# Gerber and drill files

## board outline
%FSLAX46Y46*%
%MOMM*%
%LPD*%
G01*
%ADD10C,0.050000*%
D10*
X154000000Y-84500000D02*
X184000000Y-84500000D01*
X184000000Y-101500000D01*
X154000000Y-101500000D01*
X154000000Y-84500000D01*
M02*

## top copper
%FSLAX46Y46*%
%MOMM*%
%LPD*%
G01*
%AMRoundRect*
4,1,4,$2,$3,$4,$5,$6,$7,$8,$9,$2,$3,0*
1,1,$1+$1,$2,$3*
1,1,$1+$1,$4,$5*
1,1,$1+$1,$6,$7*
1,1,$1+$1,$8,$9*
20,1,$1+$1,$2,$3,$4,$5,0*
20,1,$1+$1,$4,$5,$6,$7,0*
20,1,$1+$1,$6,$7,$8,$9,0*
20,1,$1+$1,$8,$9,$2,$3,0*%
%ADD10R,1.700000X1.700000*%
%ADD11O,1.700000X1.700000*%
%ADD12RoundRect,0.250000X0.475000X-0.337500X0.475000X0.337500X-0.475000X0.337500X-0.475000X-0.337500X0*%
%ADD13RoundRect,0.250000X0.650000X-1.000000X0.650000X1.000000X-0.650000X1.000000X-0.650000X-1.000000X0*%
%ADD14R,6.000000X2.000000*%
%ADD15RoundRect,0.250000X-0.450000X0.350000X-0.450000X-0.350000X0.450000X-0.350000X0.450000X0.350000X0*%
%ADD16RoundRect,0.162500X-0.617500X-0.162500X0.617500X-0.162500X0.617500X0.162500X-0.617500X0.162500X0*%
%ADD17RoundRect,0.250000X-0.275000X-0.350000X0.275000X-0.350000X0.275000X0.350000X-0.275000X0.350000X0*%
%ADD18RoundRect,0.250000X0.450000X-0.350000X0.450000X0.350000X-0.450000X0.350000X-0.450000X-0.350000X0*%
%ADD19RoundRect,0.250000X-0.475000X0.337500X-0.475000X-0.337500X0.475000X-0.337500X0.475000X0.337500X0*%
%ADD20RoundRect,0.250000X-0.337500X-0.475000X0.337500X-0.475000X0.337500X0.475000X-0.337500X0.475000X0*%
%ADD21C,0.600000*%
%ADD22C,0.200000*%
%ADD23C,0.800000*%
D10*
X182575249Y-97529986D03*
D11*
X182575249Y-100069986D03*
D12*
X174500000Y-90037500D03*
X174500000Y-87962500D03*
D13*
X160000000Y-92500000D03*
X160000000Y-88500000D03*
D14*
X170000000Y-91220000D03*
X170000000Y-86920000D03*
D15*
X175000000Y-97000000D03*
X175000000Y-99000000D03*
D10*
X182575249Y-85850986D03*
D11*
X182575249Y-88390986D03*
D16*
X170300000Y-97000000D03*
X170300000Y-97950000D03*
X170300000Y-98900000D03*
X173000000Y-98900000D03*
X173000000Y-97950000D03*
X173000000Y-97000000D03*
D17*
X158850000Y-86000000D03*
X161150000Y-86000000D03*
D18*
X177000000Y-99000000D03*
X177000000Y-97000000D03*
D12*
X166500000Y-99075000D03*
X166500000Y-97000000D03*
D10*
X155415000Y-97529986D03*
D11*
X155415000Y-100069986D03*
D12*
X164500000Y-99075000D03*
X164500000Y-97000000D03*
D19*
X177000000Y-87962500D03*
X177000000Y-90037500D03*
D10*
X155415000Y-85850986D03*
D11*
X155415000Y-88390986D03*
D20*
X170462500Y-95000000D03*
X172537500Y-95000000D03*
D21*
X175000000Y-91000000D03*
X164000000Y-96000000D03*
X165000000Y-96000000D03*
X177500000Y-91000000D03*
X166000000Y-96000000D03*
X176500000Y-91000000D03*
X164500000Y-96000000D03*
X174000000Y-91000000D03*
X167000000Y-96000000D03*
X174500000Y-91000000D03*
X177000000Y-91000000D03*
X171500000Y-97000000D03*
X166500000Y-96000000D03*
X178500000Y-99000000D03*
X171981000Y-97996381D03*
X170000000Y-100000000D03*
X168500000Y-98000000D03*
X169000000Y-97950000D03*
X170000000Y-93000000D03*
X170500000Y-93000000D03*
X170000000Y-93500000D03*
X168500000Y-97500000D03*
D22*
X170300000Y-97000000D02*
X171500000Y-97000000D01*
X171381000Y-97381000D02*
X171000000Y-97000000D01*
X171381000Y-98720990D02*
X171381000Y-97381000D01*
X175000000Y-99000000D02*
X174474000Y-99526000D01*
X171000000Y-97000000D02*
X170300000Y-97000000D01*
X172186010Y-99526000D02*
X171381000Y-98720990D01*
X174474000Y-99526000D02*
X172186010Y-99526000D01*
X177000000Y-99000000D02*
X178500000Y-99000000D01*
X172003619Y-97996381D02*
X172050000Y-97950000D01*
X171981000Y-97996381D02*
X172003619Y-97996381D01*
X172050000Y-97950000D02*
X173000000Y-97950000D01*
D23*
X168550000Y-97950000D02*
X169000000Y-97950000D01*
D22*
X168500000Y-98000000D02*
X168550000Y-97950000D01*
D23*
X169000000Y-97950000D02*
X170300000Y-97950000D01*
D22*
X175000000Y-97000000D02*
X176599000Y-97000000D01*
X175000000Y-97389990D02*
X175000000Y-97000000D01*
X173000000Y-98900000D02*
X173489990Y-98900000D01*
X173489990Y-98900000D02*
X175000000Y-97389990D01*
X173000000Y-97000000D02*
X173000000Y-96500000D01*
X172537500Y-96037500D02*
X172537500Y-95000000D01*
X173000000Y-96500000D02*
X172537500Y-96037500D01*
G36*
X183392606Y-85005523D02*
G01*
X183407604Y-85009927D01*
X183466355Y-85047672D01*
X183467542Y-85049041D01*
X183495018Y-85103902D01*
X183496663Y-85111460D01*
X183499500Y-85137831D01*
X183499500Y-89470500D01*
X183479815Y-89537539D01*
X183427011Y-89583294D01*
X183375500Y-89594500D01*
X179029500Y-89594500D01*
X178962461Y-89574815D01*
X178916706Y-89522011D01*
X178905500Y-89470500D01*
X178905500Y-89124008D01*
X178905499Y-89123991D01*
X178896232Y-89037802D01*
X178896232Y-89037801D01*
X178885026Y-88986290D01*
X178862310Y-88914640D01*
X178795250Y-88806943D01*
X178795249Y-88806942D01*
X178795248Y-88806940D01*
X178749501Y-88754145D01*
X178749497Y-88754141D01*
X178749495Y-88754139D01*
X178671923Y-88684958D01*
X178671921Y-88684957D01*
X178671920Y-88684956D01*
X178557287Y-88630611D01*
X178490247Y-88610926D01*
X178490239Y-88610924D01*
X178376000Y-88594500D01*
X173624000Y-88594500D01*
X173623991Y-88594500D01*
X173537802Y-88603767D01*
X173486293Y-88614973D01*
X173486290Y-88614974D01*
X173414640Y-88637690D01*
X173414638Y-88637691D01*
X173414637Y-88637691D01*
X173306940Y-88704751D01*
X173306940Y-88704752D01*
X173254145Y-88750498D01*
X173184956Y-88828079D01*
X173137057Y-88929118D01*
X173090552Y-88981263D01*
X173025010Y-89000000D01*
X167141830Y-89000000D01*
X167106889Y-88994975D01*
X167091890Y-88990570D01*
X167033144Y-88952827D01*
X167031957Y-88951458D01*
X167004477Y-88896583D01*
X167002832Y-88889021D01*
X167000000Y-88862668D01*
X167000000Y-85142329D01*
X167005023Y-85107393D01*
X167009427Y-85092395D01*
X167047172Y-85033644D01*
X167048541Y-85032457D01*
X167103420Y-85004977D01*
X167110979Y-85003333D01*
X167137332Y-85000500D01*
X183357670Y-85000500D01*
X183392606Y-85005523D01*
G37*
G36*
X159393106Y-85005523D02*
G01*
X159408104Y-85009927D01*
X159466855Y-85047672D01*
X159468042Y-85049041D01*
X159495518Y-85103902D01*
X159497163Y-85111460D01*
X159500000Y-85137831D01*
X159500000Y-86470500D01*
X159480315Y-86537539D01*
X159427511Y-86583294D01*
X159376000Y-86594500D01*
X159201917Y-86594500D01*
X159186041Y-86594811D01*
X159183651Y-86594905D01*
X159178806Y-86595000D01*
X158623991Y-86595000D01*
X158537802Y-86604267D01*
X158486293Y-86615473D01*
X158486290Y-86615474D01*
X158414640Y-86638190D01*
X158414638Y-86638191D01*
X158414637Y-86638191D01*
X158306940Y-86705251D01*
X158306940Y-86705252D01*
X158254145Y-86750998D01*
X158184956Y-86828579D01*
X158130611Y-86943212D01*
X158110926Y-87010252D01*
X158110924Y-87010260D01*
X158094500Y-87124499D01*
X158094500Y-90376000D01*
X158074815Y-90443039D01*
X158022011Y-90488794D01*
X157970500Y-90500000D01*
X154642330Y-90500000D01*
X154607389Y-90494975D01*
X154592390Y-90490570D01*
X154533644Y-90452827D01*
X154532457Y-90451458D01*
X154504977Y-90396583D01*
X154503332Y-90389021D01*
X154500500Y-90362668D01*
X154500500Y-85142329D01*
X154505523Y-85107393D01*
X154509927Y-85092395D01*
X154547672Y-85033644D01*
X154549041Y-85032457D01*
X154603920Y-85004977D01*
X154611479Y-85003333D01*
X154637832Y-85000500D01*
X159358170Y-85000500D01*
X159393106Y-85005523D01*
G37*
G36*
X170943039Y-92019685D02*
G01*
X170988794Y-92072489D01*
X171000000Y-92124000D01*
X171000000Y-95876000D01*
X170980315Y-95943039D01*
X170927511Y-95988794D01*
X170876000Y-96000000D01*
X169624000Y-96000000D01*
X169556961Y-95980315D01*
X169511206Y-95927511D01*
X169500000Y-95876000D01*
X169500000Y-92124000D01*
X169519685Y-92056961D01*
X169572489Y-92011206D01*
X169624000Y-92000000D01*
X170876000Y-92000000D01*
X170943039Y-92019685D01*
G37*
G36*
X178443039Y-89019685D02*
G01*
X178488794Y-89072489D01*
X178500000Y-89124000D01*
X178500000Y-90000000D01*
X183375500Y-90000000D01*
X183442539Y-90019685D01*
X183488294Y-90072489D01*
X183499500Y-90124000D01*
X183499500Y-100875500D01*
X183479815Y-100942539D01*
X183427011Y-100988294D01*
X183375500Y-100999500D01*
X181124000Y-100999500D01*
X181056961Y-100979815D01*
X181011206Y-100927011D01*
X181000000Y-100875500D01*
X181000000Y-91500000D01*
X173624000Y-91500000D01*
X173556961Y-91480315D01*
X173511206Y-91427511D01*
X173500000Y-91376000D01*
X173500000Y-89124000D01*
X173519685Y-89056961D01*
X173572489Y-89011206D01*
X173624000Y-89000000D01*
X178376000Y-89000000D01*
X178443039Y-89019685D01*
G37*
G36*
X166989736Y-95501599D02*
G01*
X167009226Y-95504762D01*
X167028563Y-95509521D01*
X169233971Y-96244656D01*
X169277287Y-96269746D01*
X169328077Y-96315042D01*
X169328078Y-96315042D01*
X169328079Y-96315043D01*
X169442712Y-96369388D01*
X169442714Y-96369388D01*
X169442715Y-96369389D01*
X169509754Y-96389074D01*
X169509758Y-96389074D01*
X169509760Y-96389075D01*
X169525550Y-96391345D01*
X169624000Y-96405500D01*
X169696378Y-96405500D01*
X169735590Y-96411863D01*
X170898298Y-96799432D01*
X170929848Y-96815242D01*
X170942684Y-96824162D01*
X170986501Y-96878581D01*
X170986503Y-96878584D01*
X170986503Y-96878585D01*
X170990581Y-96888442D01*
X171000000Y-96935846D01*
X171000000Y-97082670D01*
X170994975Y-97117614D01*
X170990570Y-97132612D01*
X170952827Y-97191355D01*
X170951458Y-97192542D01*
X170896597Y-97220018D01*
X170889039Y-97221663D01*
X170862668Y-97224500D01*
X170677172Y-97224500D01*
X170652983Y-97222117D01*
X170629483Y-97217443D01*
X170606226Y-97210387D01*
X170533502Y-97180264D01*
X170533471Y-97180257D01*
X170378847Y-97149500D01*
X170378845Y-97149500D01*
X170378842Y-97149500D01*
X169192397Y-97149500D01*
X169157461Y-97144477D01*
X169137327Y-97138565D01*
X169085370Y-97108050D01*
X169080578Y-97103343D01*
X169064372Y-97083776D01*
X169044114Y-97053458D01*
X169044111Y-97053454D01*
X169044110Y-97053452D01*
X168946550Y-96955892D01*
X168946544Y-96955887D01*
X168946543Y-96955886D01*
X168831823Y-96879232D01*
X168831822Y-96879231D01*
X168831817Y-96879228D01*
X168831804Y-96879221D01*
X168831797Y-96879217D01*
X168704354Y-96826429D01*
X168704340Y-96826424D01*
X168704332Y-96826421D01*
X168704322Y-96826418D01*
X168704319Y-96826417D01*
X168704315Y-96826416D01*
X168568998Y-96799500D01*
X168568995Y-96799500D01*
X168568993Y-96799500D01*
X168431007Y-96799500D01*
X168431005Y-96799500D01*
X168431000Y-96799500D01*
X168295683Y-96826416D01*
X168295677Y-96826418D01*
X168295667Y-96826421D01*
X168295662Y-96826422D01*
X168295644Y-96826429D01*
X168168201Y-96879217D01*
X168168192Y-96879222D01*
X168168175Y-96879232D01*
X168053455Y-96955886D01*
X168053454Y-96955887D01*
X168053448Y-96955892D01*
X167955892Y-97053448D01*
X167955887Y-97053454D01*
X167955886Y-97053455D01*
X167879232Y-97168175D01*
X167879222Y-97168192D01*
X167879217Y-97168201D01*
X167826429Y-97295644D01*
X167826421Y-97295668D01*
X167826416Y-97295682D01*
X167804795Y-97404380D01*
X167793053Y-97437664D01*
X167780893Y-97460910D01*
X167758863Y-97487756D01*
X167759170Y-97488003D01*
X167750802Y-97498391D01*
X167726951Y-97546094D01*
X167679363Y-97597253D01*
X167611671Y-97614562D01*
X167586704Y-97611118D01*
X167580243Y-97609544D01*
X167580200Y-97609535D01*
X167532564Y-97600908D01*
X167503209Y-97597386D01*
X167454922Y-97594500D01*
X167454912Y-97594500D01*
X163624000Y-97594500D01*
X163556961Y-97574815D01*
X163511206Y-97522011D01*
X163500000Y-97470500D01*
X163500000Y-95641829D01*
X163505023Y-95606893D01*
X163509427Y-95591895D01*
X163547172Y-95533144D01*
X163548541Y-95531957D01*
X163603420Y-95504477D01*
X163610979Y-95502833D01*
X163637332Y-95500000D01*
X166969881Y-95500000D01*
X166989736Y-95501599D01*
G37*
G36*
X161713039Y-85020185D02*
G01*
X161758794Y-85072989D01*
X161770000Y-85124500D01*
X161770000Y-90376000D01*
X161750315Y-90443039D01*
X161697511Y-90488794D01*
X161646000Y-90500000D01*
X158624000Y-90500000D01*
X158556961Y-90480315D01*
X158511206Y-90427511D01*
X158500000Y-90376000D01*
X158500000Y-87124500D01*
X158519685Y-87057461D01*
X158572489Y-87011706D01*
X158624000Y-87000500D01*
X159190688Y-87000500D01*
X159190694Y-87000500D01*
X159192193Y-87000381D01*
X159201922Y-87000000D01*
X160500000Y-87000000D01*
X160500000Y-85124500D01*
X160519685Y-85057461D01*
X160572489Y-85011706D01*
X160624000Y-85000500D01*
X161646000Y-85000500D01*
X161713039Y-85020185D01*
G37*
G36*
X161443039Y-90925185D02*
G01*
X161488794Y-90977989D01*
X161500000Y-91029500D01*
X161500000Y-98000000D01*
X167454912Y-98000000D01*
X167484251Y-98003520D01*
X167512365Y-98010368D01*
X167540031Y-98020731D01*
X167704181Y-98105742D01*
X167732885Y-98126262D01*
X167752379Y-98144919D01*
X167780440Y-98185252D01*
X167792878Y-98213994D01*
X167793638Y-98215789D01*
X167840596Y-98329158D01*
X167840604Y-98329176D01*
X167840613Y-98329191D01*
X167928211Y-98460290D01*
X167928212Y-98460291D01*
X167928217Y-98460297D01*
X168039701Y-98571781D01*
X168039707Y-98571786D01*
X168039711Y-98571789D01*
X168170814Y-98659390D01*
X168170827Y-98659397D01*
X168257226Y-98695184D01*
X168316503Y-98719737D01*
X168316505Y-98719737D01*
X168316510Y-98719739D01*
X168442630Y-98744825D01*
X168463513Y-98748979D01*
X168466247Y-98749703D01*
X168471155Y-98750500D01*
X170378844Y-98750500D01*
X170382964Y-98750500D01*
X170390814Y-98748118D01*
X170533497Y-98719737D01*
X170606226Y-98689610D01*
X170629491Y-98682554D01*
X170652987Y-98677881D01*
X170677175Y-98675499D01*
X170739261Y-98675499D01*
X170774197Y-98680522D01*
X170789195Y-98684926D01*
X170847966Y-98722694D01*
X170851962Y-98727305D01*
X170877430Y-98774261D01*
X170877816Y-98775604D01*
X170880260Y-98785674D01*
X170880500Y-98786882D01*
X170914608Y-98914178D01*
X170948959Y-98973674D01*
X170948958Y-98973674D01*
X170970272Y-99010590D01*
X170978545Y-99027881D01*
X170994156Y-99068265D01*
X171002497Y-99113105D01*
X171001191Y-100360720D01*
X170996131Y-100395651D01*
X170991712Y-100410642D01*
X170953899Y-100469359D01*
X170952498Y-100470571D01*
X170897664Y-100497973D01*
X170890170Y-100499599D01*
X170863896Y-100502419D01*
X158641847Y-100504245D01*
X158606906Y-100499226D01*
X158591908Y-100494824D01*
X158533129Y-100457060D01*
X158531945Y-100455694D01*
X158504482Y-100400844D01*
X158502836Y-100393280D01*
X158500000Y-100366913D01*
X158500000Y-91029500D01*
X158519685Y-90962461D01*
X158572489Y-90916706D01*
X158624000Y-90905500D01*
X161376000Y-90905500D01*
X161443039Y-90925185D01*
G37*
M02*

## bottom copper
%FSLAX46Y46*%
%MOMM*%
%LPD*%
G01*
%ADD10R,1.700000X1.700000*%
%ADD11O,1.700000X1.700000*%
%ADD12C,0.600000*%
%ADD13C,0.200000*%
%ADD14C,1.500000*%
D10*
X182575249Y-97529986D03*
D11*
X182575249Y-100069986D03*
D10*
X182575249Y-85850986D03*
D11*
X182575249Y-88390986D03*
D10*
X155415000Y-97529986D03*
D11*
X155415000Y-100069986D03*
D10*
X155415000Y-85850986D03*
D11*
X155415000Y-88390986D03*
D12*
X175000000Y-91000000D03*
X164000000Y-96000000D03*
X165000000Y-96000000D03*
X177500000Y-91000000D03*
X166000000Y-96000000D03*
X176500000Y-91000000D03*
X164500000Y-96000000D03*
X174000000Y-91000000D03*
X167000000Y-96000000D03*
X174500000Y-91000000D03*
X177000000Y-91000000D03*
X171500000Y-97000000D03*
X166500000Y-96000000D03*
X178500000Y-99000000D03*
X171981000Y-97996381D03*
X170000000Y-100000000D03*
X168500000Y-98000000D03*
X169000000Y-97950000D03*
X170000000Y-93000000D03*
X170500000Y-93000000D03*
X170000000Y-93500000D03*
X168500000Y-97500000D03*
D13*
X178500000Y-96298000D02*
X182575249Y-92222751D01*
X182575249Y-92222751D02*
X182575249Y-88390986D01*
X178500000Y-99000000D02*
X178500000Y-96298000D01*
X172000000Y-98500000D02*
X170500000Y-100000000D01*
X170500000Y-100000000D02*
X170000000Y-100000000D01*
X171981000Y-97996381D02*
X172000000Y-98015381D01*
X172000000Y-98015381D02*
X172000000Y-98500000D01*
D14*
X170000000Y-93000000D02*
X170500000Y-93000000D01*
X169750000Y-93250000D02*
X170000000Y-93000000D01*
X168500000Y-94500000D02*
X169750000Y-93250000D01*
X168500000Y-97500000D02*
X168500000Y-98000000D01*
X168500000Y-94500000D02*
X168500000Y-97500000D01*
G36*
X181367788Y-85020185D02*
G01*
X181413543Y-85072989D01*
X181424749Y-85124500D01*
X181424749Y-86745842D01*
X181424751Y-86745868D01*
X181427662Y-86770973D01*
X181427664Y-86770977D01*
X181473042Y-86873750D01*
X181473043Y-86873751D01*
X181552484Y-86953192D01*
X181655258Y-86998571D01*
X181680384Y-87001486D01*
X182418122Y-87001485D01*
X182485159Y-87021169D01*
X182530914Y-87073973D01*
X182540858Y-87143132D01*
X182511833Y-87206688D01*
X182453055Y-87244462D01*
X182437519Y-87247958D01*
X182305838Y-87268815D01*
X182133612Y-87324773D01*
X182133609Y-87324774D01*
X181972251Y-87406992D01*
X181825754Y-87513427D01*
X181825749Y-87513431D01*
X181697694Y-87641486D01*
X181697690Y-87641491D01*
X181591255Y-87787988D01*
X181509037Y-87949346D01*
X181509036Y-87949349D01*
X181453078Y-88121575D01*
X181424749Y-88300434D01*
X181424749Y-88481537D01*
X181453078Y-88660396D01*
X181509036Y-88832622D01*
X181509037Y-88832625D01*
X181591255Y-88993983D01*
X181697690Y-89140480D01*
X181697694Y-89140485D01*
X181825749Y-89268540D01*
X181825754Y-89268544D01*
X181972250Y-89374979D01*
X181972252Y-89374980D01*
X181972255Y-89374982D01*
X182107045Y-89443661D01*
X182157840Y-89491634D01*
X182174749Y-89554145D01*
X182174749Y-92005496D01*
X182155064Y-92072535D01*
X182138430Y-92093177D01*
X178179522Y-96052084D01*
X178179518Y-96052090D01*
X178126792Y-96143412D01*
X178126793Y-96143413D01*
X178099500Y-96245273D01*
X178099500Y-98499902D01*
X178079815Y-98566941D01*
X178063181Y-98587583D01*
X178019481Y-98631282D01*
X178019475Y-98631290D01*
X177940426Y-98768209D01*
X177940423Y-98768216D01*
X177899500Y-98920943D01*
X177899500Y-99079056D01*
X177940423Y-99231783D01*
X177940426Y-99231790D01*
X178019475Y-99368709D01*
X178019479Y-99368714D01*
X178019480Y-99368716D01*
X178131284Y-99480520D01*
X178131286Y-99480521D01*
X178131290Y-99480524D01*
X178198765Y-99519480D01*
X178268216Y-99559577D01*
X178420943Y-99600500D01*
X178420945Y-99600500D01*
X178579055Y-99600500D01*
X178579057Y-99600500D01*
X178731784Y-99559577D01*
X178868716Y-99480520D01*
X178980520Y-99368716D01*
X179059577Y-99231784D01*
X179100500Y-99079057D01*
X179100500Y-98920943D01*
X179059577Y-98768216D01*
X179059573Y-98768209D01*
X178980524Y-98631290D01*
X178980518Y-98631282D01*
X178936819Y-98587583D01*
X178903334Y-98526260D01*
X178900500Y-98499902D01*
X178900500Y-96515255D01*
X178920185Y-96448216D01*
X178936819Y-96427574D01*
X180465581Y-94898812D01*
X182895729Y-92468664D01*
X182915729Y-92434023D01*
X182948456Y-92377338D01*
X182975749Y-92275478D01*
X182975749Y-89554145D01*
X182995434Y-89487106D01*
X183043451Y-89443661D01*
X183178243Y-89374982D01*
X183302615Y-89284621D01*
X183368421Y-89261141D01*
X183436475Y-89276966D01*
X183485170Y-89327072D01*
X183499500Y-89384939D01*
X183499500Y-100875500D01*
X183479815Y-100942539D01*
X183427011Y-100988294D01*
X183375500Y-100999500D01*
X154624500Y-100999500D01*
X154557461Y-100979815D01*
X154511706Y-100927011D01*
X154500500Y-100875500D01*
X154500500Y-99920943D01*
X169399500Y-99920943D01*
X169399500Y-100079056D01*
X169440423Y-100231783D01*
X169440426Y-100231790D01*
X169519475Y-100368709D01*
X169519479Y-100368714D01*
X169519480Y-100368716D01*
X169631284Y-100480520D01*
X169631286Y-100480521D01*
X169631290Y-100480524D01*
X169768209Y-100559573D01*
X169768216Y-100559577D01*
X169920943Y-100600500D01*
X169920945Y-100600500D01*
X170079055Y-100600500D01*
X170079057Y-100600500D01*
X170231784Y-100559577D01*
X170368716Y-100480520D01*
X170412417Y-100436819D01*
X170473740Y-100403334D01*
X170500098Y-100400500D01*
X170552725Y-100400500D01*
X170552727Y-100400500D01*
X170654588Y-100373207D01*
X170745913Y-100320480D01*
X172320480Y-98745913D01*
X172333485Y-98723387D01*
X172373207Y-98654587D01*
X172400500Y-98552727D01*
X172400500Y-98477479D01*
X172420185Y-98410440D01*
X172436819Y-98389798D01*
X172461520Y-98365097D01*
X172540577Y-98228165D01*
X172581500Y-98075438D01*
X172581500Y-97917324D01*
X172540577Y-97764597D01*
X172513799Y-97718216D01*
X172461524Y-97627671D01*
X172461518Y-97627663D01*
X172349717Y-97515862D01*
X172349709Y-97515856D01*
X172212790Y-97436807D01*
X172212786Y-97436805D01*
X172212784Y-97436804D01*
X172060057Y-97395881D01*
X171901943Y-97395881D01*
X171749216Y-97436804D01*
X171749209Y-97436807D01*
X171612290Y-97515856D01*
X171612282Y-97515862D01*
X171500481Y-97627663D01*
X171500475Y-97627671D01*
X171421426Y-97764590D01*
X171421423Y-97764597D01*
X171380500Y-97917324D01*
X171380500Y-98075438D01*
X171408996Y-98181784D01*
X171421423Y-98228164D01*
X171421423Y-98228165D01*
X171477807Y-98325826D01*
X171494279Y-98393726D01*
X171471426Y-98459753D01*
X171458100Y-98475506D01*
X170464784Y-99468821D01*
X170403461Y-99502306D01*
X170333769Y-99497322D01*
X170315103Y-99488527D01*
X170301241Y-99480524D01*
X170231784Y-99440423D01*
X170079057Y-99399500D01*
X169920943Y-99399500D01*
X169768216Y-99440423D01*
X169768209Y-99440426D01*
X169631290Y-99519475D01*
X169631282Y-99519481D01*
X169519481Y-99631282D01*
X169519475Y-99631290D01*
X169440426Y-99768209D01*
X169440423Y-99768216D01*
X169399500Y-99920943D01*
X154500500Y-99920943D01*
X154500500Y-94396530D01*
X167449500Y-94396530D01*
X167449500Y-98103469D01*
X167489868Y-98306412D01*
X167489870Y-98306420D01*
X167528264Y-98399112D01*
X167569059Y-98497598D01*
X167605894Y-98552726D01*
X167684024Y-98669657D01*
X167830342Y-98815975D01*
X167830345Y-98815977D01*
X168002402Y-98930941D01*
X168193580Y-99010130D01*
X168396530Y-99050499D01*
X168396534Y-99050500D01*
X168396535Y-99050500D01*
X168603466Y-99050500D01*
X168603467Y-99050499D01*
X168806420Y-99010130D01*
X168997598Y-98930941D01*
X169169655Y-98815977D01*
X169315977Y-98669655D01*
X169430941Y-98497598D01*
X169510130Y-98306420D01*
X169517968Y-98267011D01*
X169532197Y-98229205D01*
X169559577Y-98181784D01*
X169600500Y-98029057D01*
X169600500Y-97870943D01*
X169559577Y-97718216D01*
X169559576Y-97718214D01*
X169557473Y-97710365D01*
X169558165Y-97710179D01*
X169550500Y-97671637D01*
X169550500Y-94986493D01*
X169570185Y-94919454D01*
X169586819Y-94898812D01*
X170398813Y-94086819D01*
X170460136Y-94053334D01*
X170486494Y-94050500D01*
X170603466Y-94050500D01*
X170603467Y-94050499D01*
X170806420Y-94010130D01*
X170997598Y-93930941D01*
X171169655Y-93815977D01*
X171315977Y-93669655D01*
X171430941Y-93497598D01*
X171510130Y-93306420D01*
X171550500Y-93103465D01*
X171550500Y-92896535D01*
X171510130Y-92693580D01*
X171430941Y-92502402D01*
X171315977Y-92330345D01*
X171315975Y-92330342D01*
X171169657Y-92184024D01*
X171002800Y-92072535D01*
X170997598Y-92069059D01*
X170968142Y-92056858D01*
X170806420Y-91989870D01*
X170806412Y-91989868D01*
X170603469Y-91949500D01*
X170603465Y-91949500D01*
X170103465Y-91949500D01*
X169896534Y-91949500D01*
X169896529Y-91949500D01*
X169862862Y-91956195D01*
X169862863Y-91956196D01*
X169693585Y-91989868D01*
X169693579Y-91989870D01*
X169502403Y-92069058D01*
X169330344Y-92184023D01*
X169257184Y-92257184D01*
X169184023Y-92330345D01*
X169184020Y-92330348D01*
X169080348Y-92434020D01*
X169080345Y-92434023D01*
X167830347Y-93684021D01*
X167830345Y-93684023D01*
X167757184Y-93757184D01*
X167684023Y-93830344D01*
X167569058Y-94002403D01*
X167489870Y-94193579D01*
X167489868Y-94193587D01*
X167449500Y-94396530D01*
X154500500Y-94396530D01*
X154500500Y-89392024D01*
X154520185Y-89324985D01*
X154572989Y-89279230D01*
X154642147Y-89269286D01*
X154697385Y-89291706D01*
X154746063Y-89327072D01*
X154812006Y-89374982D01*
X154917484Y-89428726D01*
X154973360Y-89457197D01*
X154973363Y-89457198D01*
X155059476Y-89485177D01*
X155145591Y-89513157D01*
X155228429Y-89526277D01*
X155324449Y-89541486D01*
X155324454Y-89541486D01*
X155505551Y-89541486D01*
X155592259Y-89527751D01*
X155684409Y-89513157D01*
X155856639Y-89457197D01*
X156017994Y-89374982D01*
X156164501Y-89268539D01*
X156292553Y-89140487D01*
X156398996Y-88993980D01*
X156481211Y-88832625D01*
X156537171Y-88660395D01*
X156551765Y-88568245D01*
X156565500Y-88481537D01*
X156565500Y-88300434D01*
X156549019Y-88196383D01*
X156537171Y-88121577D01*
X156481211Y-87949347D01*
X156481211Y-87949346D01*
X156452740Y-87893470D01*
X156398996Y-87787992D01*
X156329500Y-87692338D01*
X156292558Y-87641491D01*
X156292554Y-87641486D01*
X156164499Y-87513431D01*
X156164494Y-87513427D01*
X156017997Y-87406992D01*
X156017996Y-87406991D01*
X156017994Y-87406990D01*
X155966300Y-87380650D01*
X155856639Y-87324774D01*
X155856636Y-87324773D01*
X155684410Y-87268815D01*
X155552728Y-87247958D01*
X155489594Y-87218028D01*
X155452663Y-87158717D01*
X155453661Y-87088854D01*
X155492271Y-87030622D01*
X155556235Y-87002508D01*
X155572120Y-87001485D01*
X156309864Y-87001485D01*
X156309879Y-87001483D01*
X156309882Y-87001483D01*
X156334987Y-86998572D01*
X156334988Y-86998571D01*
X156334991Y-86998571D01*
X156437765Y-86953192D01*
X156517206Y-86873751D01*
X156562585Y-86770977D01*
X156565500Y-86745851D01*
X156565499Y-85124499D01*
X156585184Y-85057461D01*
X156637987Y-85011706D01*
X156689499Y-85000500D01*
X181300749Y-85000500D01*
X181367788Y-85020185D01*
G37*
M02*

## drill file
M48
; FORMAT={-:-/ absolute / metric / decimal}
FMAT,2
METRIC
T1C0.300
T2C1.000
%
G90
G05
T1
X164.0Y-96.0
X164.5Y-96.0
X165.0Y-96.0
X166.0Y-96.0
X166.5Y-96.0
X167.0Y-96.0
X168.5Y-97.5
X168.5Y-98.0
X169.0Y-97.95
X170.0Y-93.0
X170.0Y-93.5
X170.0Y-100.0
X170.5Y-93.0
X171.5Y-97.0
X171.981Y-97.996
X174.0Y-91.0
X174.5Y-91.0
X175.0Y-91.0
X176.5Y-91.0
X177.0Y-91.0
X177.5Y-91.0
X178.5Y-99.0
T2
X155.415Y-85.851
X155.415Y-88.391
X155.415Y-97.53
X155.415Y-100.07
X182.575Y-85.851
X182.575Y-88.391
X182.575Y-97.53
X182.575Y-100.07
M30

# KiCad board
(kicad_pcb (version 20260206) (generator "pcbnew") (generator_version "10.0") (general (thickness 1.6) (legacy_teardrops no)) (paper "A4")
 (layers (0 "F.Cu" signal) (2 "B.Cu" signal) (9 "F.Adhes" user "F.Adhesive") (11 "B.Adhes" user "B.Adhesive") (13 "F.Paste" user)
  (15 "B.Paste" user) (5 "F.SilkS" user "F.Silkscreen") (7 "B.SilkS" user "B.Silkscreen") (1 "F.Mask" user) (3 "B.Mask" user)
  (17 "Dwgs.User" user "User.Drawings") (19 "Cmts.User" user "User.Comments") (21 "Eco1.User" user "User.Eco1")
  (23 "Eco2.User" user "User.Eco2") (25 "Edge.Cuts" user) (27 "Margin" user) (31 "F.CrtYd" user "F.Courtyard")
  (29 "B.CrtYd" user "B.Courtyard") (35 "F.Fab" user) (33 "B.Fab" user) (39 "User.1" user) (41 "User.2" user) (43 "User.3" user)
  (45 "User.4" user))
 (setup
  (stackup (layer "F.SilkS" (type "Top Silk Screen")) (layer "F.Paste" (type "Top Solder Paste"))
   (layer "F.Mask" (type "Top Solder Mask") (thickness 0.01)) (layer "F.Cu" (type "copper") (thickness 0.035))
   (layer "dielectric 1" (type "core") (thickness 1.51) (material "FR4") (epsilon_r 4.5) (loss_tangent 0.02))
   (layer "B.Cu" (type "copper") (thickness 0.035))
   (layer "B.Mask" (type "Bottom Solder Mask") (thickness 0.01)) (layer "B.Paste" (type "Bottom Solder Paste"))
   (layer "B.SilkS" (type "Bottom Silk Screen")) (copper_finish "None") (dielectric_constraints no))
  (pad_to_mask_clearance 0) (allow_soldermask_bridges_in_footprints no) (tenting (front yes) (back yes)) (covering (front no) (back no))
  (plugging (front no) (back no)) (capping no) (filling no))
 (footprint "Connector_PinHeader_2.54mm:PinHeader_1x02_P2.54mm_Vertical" (layer "F.Cu") (at 182.575249 97.529986)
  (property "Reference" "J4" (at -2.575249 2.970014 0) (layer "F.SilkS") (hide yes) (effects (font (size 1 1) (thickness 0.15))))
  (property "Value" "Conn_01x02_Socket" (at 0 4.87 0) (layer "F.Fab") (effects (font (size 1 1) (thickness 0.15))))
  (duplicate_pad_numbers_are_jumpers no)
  (pad "1" thru_hole rect (at 0 0) (size 1.7 1.7) (drill 1) (layers "*.Cu" "*.Mask") (remove_unused_layers no) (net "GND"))
  (pad "2" thru_hole oval (at 0 2.54) (size 1.7 1.7) (drill 1) (layers "*.Cu" "*.Mask") (remove_unused_layers no) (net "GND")))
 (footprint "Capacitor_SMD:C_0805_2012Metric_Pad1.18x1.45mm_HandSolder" (layer "F.Cu") (at 174.5 89 90)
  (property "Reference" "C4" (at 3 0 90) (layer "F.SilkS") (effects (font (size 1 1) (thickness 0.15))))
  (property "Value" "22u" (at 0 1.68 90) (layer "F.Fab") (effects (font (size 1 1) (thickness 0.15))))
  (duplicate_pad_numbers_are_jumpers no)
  (pad "1" smd roundrect (at -1.0375 0 90) (size 1.175 1.45) (layers "F.Cu" "F.Mask" "F.Paste") (roundrect_rratio 0.212766) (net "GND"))
  (pad "2" smd roundrect (at 1.0375 0 90) (size 1.175 1.45) (layers "F.Cu" "F.Mask" "F.Paste") (roundrect_rratio 0.212766) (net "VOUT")))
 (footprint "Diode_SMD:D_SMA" (layer "F.Cu") (at 160 90.5 90)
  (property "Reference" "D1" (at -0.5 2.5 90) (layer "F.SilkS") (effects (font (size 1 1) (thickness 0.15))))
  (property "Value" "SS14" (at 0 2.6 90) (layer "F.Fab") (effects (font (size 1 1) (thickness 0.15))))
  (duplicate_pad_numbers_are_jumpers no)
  (pad "1" smd roundrect (at -2 0 90) (size 2.5 1.8) (layers "F.Cu" "F.Mask" "F.Paste") (roundrect_rratio 0.1388888889) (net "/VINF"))
  (pad "2" smd roundrect (at 2 0 90) (size 2.5 1.8) (layers "F.Cu" "F.Mask" "F.Paste") (roundrect_rratio 0.1388888889) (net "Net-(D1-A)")))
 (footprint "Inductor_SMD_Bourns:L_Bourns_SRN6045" (layer "F.Cu") (at 170 89.075 90)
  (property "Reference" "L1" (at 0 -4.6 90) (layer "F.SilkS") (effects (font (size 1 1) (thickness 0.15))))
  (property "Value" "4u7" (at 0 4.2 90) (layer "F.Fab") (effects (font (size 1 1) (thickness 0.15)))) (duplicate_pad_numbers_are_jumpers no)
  (pad "1" smd rect (at -2.145 0 90) (size 2 6) (layers "F.Cu" "F.Mask" "F.Paste") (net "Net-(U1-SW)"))
  (pad "2" smd rect (at 2.155 0 90) (size 2 6) (layers "F.Cu" "F.Mask" "F.Paste") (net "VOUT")))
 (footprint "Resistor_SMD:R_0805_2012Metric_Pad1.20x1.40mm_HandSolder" (layer "F.Cu") (at 175 98 -90)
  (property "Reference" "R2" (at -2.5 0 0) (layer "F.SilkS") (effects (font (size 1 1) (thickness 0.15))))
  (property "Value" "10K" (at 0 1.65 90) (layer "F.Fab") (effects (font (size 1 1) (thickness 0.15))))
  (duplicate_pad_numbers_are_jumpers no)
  (pad "1" smd roundrect (at -1 0 270) (size 1.2 1.4) (layers "F.Cu" "F.Mask" "F.Paste") (roundrect_rratio 0.208333) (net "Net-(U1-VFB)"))
  (pad "2" smd roundrect (at 1 0 270) (size 1.2 1.4) (layers "F.Cu" "F.Mask" "F.Paste") (roundrect_rratio 0.208333) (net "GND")))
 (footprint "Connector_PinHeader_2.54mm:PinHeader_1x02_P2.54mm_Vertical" (layer "F.Cu") (at 182.575249 85.850986)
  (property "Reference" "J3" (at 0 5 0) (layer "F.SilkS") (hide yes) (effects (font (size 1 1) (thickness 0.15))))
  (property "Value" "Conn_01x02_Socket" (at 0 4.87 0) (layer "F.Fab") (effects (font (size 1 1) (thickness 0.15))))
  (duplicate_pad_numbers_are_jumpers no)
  (pad "1" thru_hole rect (at 0 0) (size 1.7 1.7) (drill 1) (layers "*.Cu" "*.Mask") (remove_unused_layers no) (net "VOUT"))
  (pad "2" thru_hole oval (at 0 2.54) (size 1.7 1.7) (drill 1) (layers "*.Cu" "*.Mask") (remove_unused_layers no) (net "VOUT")))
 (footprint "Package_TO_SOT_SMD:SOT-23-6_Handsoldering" (layer "F.Cu") (at 171.65 97.95)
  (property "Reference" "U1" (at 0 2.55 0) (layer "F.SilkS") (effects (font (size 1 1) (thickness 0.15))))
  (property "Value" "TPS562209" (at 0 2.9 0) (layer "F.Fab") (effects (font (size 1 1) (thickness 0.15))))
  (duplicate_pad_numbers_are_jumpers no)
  (pad "1" smd roundrect (at -1.35 -0.95) (size 1.56 0.65) (layers "F.Cu" "F.Mask" "F.Paste") (roundrect_rratio 0.25) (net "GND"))
  (pad "2" smd roundrect (at -1.35 0) (size 1.56 0.65) (layers "F.Cu" "F.Mask" "F.Paste") (roundrect_rratio 0.25) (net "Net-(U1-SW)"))
  (pad "3" smd roundrect (at -1.35 0.95) (size 1.56 0.65) (layers "F.Cu" "F.Mask" "F.Paste") (roundrect_rratio 0.25) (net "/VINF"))
  (pad "4" smd roundrect (at 1.35 0.95) (size 1.56 0.65) (layers "F.Cu" "F.Mask" "F.Paste") (roundrect_rratio 0.25) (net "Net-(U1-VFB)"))
  (pad "5" smd roundrect (at 1.35 0) (size 1.56 0.65) (layers "F.Cu" "F.Mask" "F.Paste") (roundrect_rratio 0.25) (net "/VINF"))
  (pad "6" smd roundrect (at 1.35 -0.95) (size 1.56 0.65) (layers "F.Cu" "F.Mask" "F.Paste") (roundrect_rratio 0.25) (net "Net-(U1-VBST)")))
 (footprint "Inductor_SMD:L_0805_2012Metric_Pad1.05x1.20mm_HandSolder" (layer "F.Cu") (at 160 86)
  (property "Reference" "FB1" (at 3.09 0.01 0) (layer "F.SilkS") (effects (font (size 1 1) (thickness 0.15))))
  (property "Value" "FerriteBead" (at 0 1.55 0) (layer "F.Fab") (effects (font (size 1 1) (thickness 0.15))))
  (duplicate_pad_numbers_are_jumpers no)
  (pad "1" smd roundrect (at -1.15 0) (size 1.05 1.2) (layers "F.Cu" "F.Mask" "F.Paste") (roundrect_rratio 0.238095) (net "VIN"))
  (pad "2" smd roundrect (at 1.15 0) (size 1.05 1.2) (layers "F.Cu" "F.Mask" "F.Paste") (roundrect_rratio 0.238095) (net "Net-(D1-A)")))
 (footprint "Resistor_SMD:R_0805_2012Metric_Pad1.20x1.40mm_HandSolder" (layer "F.Cu") (at 177 98 90)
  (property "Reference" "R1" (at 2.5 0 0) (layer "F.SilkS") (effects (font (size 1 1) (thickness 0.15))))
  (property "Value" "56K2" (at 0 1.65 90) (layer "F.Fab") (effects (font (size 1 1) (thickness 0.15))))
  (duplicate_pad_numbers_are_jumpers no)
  (pad "1" smd roundrect (at -1 0 90) (size 1.2 1.4) (layers "F.Cu" "F.Mask" "F.Paste") (roundrect_rratio 0.208333) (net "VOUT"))
  (pad "2" smd roundrect (at 1 0 90) (size 1.2 1.4) (layers "F.Cu" "F.Mask" "F.Paste") (roundrect_rratio 0.208333) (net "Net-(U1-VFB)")))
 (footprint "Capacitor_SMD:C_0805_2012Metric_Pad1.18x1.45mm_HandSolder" (layer "F.Cu") (at 166.5 98.0375 90)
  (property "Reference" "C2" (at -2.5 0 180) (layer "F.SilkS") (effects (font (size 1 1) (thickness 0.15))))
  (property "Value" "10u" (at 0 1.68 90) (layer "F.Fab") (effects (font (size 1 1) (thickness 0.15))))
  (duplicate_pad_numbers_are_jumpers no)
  (pad "1" smd roundrect (at -1.0375 0 90) (size 1.175 1.45) (layers "F.Cu" "F.Mask" "F.Paste") (roundrect_rratio 0.212766) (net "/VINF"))
  (pad "2" smd roundrect (at 1.0375 0 90) (size 1.175 1.45) (layers "F.Cu" "F.Mask" "F.Paste") (roundrect_rratio 0.212766) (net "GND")))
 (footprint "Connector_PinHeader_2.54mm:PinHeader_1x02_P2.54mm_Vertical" (layer "F.Cu") (at 155.415 97.529986)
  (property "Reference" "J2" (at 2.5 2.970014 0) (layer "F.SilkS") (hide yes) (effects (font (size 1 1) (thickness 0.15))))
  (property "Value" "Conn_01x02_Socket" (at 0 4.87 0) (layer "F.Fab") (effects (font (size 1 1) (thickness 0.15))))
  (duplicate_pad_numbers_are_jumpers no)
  (pad "1" thru_hole rect (at 0 0) (size 1.7 1.7) (drill 1) (layers "*.Cu" "*.Mask") (remove_unused_layers no) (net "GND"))
  (pad "2" thru_hole oval (at 0 2.54) (size 1.7 1.7) (drill 1) (layers "*.Cu" "*.Mask") (remove_unused_layers no) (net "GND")))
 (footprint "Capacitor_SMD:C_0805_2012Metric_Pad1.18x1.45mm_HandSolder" (layer "F.Cu") (at 164.5 98.0375 90)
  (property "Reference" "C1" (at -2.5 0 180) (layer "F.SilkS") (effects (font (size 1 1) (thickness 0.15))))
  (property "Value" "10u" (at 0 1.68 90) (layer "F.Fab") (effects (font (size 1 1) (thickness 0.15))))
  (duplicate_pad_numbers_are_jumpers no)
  (pad "1" smd roundrect (at -1.0375 0 90) (size 1.175 1.45) (layers "F.Cu" "F.Mask" "F.Paste") (roundrect_rratio 0.212766) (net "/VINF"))
  (pad "2" smd roundrect (at 1.0375 0 90) (size 1.175 1.45) (layers "F.Cu" "F.Mask" "F.Paste") (roundrect_rratio 0.212766) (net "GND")))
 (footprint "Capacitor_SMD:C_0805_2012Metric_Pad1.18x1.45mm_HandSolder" (layer "F.Cu") (at 177 89 -90)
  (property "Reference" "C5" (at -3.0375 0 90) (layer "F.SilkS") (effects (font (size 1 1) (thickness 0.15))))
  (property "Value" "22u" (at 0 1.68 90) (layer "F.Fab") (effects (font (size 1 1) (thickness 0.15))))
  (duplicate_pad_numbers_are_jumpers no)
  (pad "1" smd roundrect (at -1.0375 0 270) (size 1.175 1.45) (layers "F.Cu" "F.Mask" "F.Paste") (roundrect_rratio 0.212766) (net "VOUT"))
  (pad "2" smd roundrect (at 1.0375 0 270) (size 1.175 1.45) (layers "F.Cu" "F.Mask" "F.Paste") (roundrect_rratio 0.212766) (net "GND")))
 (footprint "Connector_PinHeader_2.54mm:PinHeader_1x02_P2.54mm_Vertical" (layer "F.Cu") (at 155.415 85.850986)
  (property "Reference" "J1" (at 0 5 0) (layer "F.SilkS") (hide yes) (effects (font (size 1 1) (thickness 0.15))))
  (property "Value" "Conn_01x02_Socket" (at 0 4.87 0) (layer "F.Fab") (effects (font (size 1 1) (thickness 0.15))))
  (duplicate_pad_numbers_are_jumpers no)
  (pad "1" thru_hole rect (at 0 0) (size 1.7 1.7) (drill 1) (layers "*.Cu" "*.Mask") (remove_unused_layers no) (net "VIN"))
  (pad "2" thru_hole oval (at 0 2.54) (size 1.7 1.7) (drill 1) (layers "*.Cu" "*.Mask") (remove_unused_layers no) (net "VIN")))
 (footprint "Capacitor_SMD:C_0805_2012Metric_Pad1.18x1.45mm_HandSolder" (layer "F.Cu") (at 171.5 95)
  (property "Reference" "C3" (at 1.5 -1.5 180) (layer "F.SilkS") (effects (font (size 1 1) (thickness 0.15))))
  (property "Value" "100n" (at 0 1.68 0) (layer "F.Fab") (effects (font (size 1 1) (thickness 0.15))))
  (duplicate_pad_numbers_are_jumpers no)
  (pad "1" smd roundrect (at -1.0375 0) (size 1.175 1.45) (layers "F.Cu" "F.Mask" "F.Paste") (roundrect_rratio 0.212766) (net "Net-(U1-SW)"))
  (pad "2" smd roundrect (at 1.0375 0) (size 1.175 1.45) (layers "F.Cu" "F.Mask" "F.Paste") (roundrect_rratio 0.212766)
   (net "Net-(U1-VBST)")))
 (gr_rect (start 154 84.5) (end 184 101.5) (stroke (width 0.05) (type default)) (fill no) (layer "Edge.Cuts"))
 (segment (start 170.3 97) (end 171.5 97) (width 0.2) (layer "F.Cu") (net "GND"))
 (segment (start 171.381 97.381) (end 171 97) (width 0.2) (layer "F.Cu") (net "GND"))
 (segment (start 171.381 98.72099) (end 171.381 97.381) (width 0.2) (layer "F.Cu") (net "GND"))
 (segment (start 175 99) (end 174.474 99.526) (width 0.2) (layer "F.Cu") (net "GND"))
 (segment (start 171 97) (end 170.3 97) (width 0.2) (layer "F.Cu") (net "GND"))
 (segment (start 172.18601 99.526) (end 171.381 98.72099) (width 0.2) (layer "F.Cu") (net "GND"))
 (segment (start 174.474 99.526) (end 172.18601 99.526) (width 0.2) (layer "F.Cu") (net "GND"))
 (via (at 175 91) (size 0.6) (drill 0.3) (layers "F.Cu" "B.Cu") (free yes) (capping no) (covering (front no) (back no))
  (plugging (front no) (back no)) (filling no) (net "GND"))
 (via (at 164 96) (size 0.6) (drill 0.3) (layers "F.Cu" "B.Cu") (free yes) (capping no) (covering (front no) (back no))
  (plugging (front no) (back no)) (filling no) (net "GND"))
 (via (at 165 96) (size 0.6) (drill 0.3) (layers "F.Cu" "B.Cu") (free yes) (capping no) (covering (front no) (back no))
  (plugging (front no) (back no)) (filling no) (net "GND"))
 (via (at 177.5 91) (size 0.6) (drill 0.3) (layers "F.Cu" "B.Cu") (free yes) (capping no) (covering (front no) (back no))
  (plugging (front no) (back no)) (filling no) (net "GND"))
 (via (at 166 96) (size 0.6) (drill 0.3) (layers "F.Cu" "B.Cu") (free yes) (capping no) (covering (front no) (back no))
  (plugging (front no) (back no)) (filling no) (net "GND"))
 (via (at 176.5 91) (size 0.6) (drill 0.3) (layers "F.Cu" "B.Cu") (free yes) (capping no) (covering (front no) (back no))
  (plugging (front no) (back no)) (filling no) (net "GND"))
 (via (at 164.5 96) (size 0.6) (drill 0.3) (layers "F.Cu" "B.Cu") (free yes) (capping no) (covering (front no) (back no))
  (plugging (front no) (back no)) (filling no) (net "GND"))
 (via (at 174 91) (size 0.6) (drill 0.3) (layers "F.Cu" "B.Cu") (free yes) (capping no) (covering (front no) (back no))
  (plugging (front no) (back no)) (filling no) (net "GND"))
 (via (at 167 96) (size 0.6) (drill 0.3) (layers "F.Cu" "B.Cu") (free yes) (capping no) (covering (front no) (back no))
  (plugging (front no) (back no)) (filling no) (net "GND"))
 (via (at 174.5 91) (size 0.6) (drill 0.3) (layers "F.Cu" "B.Cu") (free yes) (capping no) (covering (front no) (back no))
  (plugging (front no) (back no)) (filling no) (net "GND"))
 (via (at 177 91) (size 0.6) (drill 0.3) (layers "F.Cu" "B.Cu") (free yes) (capping no) (covering (front no) (back no))
  (plugging (front no) (back no)) (filling no) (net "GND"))
 (via (at 171.5 97) (size 0.6) (drill 0.3) (layers "F.Cu" "B.Cu") (capping no) (covering (front no) (back no))
  (plugging (front no) (back no)) (filling no) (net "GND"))
 (via (at 166.5 96) (size 0.6) (drill 0.3) (layers "F.Cu" "B.Cu") (free yes) (capping no) (covering (front no) (back no))
  (plugging (front no) (back no)) (filling no) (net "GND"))
 (segment (start 177 99) (end 178.5 99) (width 0.2) (layer "F.Cu") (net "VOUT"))
 (via (at 178.5 99) (size 0.6) (drill 0.3) (layers "F.Cu" "B.Cu") (capping no) (covering (front no) (back no))
  (plugging (front no) (back no)) (filling no) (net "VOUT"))
 (segment (start 178.5 96.298) (end 182.575249 92.222751) (width 0.2) (layer "B.Cu") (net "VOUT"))
 (segment (start 182.575249 92.222751) (end 182.575249 88.390986) (width 0.2) (layer "B.Cu") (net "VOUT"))
 (segment (start 178.5 99) (end 178.5 96.298) (width 0.2) (layer "B.Cu") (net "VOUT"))
 (segment (start 172.003619 97.996381) (end 172.05 97.95) (width 0.2) (layer "F.Cu") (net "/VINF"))
 (segment (start 171.981 97.996381) (end 172.003619 97.996381) (width 0.2) (layer "F.Cu") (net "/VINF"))
 (segment (start 172.05 97.95) (end 173 97.95) (width 0.2) (layer "F.Cu") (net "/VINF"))
 (via (at 171.981 97.996381) (size 0.6) (drill 0.3) (layers "F.Cu" "B.Cu") (capping no) (covering (front no) (back no))
  (plugging (front no) (back no)) (filling no) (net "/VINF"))
 (via (at 170 100) (size 0.6) (drill 0.3) (layers "F.Cu" "B.Cu") (capping no) (covering (front no) (back no))
  (plugging (front no) (back no)) (filling no) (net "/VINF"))
 (segment (start 172 98.5) (end 170.5 100) (width 0.2) (layer "B.Cu") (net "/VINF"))
 (segment (start 170.5 100) (end 170 100) (width 0.2) (layer "B.Cu") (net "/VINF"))
 (segment (start 171.981 97.996381) (end 172 98.015381) (width 0.2) (layer "B.Cu") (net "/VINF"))
 (segment (start 172 98.015381) (end 172 98.5) (width 0.2) (layer "B.Cu") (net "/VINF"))
 (segment (start 168.55 97.95) (end 169 97.95) (width 0.8) (layer "F.Cu") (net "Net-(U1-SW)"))
 (segment (start 168.5 98) (end 168.55 97.95) (width 0.2) (layer "F.Cu") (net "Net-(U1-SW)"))
 (segment (start 169 97.95) (end 170.3 97.95) (width 0.8) (layer "F.Cu") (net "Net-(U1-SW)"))
 (via (at 168.5 98) (size 0.6) (drill 0.3) (layers "F.Cu" "B.Cu") (capping no) (covering (front no) (back no))
  (plugging (front no) (back no)) (filling no) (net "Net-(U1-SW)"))
 (via (at 169 97.95) (size 0.6) (drill 0.3) (layers "F.Cu" "B.Cu") (capping no) (covering (front no) (back no))
  (plugging (front no) (back no)) (filling no) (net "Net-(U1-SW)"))
 (via (at 170 93) (size 0.6) (drill 0.3) (layers "F.Cu" "B.Cu") (capping no) (covering (front no) (back no)) (plugging (front no) (back no))
  (filling no) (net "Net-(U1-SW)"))
 (via (at 170.5 93) (size 0.6) (drill 0.3) (layers "F.Cu" "B.Cu") (capping no) (covering (front no) (back no))
  (plugging (front no) (back no)) (filling no) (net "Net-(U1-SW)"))
 (via (at 170 93.5) (size 0.6) (drill 0.3) (layers "F.Cu" "B.Cu") (capping no) (covering (front no) (back no))
  (plugging (front no) (back no)) (filling no) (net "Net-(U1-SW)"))
 (via (at 168.5 97.5) (size 0.6) (drill 0.3) (layers "F.Cu" "B.Cu") (capping no) (covering (front no) (back no))
  (plugging (front no) (back no)) (filling no) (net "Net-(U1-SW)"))
 (segment (start 170 93) (end 170.5 93) (width 1.5) (layer "B.Cu") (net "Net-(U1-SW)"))
 (segment (start 169.75 93.25) (end 170 93) (width 1.5) (layer "B.Cu") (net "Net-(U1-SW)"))
 (segment (start 168.5 94.5) (end 169.75 93.25) (width 1.5) (layer "B.Cu") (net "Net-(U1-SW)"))
 (segment (start 168.5 97.5) (end 168.5 98) (width 1.5) (layer "B.Cu") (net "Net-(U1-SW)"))
 (segment (start 168.5 94.5) (end 168.5 97.5) (width 1.5) (layer "B.Cu") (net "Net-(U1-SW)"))
 (segment (start 175 97) (end 176.599 97) (width 0.2) (layer "F.Cu") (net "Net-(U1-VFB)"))
 (segment (start 175 97.38999) (end 175 97) (width 0.2) (layer "F.Cu") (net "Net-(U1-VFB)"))
 (segment (start 173 98.9) (end 173.48999 98.9) (width 0.2) (layer "F.Cu") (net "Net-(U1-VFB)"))
 (segment (start 173.48999 98.9) (end 175 97.38999) (width 0.2) (layer "F.Cu") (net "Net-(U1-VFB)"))
 (segment (start 173 97) (end 173 96.5) (width 0.2) (layer "F.Cu") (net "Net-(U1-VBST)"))
 (segment (start 172.5375 96.0375) (end 172.5375 95) (width 0.2) (layer "F.Cu") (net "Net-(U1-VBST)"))
 (segment (start 173 96.5) (end 172.5375 96.0375) (width 0.2) (layer "F.Cu") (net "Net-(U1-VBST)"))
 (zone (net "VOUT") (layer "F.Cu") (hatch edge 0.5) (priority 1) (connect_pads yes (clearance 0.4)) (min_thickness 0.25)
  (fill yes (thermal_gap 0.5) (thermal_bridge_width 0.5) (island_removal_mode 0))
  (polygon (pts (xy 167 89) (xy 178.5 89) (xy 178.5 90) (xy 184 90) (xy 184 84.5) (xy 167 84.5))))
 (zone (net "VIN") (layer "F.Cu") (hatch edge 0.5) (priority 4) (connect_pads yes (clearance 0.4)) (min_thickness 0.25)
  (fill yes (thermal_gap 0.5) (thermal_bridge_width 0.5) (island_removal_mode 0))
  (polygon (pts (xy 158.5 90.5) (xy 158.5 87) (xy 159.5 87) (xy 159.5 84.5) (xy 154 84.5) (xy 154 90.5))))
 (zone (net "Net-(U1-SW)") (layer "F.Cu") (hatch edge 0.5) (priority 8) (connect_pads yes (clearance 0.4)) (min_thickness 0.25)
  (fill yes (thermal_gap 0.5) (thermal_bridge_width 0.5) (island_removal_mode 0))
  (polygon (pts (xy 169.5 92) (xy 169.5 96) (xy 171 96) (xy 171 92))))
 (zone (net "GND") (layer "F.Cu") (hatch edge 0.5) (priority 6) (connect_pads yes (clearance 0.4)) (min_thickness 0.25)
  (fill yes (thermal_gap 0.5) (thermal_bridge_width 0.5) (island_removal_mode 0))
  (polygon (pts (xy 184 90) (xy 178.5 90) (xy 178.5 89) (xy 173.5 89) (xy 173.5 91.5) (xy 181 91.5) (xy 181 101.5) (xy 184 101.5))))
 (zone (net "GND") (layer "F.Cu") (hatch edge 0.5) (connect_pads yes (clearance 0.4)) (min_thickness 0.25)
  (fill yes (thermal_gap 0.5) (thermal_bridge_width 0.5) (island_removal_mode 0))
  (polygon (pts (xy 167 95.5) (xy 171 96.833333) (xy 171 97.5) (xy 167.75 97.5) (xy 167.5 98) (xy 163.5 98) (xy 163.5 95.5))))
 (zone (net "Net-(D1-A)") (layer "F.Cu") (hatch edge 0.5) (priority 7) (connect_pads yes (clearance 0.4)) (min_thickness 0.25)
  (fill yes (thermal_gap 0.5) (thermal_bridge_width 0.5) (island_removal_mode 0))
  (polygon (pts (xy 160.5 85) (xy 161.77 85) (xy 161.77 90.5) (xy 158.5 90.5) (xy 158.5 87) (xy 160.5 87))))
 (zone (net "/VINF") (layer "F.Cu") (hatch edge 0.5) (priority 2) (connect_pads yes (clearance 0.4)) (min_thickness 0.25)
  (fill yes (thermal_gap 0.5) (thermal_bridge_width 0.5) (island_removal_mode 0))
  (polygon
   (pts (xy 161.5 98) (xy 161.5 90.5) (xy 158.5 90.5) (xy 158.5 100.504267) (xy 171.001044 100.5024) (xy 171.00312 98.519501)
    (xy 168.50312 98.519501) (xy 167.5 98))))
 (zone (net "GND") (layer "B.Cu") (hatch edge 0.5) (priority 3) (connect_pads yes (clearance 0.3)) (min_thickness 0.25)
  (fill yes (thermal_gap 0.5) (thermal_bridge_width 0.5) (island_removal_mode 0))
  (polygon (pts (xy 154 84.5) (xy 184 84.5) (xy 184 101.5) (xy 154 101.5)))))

